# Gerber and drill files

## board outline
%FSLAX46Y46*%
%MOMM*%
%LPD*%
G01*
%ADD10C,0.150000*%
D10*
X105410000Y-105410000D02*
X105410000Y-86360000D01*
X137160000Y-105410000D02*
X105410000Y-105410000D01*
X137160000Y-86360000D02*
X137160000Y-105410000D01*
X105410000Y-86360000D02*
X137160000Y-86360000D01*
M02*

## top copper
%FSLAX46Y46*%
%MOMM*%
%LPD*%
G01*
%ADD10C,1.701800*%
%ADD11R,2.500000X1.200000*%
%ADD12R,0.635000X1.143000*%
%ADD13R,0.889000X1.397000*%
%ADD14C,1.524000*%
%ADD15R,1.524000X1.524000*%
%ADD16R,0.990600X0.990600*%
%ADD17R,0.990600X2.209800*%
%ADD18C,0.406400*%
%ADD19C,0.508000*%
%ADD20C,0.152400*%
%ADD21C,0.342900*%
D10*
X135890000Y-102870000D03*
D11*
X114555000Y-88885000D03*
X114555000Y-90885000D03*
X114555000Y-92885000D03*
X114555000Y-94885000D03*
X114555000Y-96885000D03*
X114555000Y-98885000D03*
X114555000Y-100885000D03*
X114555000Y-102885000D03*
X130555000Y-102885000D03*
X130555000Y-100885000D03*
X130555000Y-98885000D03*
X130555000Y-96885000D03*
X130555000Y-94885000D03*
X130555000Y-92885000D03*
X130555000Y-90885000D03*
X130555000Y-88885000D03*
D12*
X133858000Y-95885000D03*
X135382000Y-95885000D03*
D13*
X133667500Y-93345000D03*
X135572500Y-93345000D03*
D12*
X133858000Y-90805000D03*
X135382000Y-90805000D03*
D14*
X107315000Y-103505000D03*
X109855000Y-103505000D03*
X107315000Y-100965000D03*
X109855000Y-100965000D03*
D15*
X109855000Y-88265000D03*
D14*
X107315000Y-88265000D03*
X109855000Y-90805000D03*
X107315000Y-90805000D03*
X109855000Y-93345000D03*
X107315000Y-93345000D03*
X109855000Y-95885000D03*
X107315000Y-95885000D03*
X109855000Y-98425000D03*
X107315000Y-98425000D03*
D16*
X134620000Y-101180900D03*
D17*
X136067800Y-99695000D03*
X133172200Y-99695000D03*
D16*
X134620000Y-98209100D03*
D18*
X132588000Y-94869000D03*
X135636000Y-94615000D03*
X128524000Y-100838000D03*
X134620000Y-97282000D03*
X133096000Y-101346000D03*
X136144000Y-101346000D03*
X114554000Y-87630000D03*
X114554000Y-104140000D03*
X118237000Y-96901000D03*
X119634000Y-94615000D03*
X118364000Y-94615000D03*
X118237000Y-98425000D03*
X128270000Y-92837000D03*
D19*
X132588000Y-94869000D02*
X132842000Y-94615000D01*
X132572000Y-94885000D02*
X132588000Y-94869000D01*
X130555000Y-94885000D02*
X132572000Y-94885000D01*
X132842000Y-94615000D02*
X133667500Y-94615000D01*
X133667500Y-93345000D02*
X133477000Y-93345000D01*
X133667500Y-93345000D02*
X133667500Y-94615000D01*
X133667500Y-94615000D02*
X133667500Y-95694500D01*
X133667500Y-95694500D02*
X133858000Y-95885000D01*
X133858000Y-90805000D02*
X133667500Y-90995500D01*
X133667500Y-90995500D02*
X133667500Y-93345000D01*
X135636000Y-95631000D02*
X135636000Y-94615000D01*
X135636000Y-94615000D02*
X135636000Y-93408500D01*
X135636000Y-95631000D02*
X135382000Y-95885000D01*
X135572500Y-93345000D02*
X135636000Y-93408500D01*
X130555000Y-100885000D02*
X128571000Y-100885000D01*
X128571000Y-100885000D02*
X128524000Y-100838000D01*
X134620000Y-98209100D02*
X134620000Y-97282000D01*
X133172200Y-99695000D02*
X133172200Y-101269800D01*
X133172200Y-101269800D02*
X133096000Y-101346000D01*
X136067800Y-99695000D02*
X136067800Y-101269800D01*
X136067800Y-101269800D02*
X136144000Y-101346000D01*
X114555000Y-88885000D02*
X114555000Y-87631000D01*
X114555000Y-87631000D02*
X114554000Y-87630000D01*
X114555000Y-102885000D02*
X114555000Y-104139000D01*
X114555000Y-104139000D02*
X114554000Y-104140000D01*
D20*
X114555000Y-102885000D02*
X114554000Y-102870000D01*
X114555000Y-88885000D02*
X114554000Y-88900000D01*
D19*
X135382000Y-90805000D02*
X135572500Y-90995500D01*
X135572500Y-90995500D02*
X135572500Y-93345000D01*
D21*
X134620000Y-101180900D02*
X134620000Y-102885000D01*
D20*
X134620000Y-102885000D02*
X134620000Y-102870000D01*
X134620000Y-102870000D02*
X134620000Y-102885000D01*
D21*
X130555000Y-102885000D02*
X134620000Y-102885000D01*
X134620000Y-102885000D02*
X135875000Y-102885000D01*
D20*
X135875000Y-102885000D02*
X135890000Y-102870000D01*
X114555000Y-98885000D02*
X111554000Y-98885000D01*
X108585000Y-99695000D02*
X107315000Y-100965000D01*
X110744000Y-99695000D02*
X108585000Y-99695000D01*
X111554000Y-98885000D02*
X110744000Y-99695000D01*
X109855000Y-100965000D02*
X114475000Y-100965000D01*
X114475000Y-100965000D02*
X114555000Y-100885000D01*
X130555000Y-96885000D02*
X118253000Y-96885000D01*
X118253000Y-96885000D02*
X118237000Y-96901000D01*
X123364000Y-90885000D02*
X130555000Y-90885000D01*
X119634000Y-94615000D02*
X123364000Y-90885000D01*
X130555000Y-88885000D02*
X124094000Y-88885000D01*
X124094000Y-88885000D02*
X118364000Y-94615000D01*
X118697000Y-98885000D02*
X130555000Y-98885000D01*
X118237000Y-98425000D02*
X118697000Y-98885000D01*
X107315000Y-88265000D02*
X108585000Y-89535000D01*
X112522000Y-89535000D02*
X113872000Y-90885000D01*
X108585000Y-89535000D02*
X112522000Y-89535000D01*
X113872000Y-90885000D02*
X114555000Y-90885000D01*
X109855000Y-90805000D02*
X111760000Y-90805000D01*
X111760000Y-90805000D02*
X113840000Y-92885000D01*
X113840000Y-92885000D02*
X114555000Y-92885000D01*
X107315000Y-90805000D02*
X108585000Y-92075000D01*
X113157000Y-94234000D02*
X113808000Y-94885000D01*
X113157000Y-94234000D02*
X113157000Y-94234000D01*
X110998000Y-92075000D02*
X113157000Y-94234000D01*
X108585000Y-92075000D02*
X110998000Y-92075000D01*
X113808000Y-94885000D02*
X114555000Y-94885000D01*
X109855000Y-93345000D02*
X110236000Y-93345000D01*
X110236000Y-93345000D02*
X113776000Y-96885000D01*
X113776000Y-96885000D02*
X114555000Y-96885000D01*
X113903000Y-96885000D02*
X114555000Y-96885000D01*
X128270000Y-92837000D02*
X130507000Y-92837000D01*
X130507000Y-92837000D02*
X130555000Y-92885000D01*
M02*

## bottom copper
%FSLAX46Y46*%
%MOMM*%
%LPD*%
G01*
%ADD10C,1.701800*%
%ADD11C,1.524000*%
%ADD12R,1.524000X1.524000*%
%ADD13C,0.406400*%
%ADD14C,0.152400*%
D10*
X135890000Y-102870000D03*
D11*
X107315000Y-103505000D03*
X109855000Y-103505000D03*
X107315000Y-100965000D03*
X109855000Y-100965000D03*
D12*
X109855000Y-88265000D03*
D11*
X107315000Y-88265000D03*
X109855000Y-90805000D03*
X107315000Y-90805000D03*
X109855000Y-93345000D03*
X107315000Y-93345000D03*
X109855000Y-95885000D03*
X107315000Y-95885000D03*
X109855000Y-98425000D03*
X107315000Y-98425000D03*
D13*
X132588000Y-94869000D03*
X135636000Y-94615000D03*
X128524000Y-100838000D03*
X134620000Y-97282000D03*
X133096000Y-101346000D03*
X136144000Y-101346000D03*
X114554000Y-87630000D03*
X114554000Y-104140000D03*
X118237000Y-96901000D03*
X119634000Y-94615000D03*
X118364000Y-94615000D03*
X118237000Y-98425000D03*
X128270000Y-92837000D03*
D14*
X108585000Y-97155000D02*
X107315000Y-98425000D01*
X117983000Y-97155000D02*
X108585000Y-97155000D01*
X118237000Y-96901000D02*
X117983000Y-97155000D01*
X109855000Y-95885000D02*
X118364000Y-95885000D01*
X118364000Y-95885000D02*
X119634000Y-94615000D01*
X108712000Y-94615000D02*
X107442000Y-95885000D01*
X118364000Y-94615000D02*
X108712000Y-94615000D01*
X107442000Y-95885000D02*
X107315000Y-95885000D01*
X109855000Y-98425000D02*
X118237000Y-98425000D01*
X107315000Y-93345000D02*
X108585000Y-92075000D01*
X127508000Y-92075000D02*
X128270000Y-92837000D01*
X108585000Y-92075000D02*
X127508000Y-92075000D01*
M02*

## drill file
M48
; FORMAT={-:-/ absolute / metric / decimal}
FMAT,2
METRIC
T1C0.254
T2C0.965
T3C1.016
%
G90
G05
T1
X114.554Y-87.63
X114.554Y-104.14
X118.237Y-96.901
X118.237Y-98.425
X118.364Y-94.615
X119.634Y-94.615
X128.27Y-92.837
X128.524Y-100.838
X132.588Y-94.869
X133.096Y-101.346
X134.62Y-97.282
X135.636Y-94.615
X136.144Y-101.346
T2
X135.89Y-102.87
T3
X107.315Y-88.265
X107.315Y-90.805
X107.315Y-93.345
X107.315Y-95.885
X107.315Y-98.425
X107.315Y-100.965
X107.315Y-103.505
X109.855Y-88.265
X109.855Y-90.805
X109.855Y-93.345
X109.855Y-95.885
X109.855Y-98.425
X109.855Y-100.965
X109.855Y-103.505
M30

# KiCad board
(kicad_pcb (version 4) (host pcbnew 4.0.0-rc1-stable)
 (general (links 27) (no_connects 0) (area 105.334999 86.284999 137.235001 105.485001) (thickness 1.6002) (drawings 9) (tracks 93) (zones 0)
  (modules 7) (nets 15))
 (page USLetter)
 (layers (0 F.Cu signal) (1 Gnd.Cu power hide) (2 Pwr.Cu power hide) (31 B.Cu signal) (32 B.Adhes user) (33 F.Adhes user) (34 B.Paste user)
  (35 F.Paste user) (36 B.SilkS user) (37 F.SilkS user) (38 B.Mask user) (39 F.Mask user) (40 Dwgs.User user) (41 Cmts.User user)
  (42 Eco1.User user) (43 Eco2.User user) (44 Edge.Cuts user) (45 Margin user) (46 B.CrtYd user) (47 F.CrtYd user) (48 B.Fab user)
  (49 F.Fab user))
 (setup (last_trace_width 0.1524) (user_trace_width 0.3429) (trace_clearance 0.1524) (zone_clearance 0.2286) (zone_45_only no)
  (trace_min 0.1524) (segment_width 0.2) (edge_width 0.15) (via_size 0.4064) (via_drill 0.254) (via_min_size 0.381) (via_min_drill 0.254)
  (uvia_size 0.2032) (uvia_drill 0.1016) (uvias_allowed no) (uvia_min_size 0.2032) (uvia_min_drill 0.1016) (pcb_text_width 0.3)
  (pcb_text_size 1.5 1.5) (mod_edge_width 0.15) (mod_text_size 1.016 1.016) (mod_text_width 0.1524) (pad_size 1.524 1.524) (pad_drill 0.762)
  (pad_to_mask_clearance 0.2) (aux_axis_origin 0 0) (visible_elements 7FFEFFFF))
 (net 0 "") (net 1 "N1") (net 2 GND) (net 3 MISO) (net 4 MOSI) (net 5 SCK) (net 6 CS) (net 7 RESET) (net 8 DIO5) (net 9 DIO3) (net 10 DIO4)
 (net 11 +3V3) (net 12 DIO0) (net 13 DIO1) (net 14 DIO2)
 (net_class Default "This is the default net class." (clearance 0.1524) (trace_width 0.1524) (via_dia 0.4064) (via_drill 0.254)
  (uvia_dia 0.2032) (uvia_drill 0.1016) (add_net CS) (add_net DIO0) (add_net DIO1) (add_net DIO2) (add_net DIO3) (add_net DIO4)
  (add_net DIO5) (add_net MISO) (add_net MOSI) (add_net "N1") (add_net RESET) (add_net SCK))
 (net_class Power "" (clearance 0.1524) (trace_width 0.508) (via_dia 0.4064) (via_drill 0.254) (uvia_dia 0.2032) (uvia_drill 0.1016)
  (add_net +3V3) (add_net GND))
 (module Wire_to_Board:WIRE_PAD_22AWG (layer F.Cu) (at 135.89 102.87)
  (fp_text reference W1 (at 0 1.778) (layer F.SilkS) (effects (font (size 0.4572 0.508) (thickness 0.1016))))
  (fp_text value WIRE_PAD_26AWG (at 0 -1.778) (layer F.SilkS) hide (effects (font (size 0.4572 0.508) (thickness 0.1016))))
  (pad 1 thru_hole circle (at 0 0) (size 1.7018 1.7018) (drill 0.9652) (layers *.Cu *.Mask F.SilkS) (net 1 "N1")))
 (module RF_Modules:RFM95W (layer F.Cu) (at 122.555 95.885)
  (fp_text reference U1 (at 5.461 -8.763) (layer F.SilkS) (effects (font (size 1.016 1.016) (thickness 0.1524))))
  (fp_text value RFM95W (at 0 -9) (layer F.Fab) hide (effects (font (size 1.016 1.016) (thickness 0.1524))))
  (pad 1 smd rect (at -8 -7) (size 2.5 1.2) (layers F.Cu F.Paste F.Mask) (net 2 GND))
  (pad 2 smd rect (at -8 -5) (size 2.5 1.2) (layers F.Cu F.Paste F.Mask) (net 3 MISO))
  (pad 3 smd rect (at -8 -3) (size 2.5 1.2) (layers F.Cu F.Paste F.Mask) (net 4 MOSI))
  (pad 4 smd rect (at -8 -1) (size 2.5 1.2) (layers F.Cu F.Paste F.Mask) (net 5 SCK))
  (pad 5 smd rect (at -8 1) (size 2.5 1.2) (layers F.Cu F.Paste F.Mask) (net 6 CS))
  (pad 6 smd rect (at -8 3) (size 2.5 1.2) (layers F.Cu F.Paste F.Mask) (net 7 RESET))
  (pad 7 smd rect (at -8 5) (size 2.5 1.2) (layers F.Cu F.Paste F.Mask) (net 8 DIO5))
  (pad 8 smd rect (at -8 7) (size 2.5 1.2) (layers F.Cu F.Paste F.Mask) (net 2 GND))
  (pad 9 smd rect (at 8 7) (size 2.5 1.2) (layers F.Cu F.Paste F.Mask) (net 1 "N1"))
  (pad 10 smd rect (at 8 5) (size 2.5 1.2) (layers F.Cu F.Paste F.Mask) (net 2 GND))
  (pad 11 smd rect (at 8 3) (size 2.5 1.2) (layers F.Cu F.Paste F.Mask) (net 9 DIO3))
  (pad 12 smd rect (at 8 1) (size 2.5 1.2) (layers F.Cu F.Paste F.Mask) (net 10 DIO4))
  (pad 13 smd rect (at 8 -1) (size 2.5 1.2) (layers F.Cu F.Paste F.Mask) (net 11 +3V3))
  (pad 14 smd rect (at 8 -3) (size 2.5 1.2) (layers F.Cu F.Paste F.Mask) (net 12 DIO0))
  (pad 15 smd rect (at 8 -5) (size 2.5 1.2) (layers F.Cu F.Paste F.Mask) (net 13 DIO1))
  (pad 16 smd rect (at 8 -7) (size 2.5 1.2) (layers F.Cu F.Paste F.Mask) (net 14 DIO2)))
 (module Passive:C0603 (layer F.Cu) (at 134.62 95.885)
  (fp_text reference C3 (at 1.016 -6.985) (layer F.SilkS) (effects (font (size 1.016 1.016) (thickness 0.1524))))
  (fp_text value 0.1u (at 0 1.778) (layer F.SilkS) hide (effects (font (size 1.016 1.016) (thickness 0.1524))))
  (pad 1 smd rect (at -0.762 0) (size 0.635 1.143) (layers F.Cu F.Paste F.Mask) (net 11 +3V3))
  (pad 2 smd rect (at 0.762 0) (size 0.635 1.143) (layers F.Cu F.Paste F.Mask) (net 2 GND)))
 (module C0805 (layer F.Cu) (at 134.62 93.345)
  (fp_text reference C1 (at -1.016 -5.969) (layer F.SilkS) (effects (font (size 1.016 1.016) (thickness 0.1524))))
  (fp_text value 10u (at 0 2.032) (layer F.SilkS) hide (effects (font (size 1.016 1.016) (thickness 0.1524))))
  (pad 1 smd rect (at -0.9525 0) (size 0.889 1.397) (layers F.Cu F.Paste F.Mask) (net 11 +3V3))
  (pad 2 smd rect (at 0.9525 0) (size 0.889 1.397) (layers F.Cu F.Paste F.Mask) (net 2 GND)))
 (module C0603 (layer F.Cu) (at 134.62 90.805)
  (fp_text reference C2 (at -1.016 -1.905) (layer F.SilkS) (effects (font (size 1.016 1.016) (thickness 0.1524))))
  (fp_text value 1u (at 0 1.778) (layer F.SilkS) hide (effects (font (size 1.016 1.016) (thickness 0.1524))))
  (pad 1 smd rect (at -0.762 0) (size 0.635 1.143) (layers F.Cu F.Paste F.Mask) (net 11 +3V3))
  (pad 2 smd rect (at 0.762 0) (size 0.635 1.143) (layers F.Cu F.Paste F.Mask) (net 2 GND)))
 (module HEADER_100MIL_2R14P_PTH (layer B.Cu) (at 108.585 95.885 270)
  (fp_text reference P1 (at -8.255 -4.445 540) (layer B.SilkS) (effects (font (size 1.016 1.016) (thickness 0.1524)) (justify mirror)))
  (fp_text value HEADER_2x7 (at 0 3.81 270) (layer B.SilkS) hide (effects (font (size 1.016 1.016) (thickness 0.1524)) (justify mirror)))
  (pad 14 thru_hole circle (at 7.62 1.27 270) (size 1.524 1.524) (drill 1.016) (layers *.Cu *.Mask B.SilkS) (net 2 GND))
  (pad 13 thru_hole circle (at 7.62 -1.27 270) (size 1.524 1.524) (drill 1.016) (layers *.Cu *.Mask B.SilkS) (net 11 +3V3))
  (pad 12 thru_hole circle (at 5.08 1.27 270) (size 1.524 1.524) (drill 1.016) (layers *.Cu *.Mask B.SilkS) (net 7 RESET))
  (pad 11 thru_hole circle (at 5.08 -1.27 270) (size 1.524 1.524) (drill 1.016) (layers *.Cu *.Mask B.SilkS) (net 8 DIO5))
  (pad 1 thru_hole rect (at -7.62 -1.27 270) (size 1.524 1.524) (drill 1.016) (layers *.Cu *.Mask B.SilkS) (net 2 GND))
  (pad 2 thru_hole circle (at -7.62 1.27 270) (size 1.524 1.524) (drill 1.016) (layers *.Cu *.Mask B.SilkS) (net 3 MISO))
  (pad 3 thru_hole circle (at -5.08 -1.27 270) (size 1.524 1.524) (drill 1.016) (layers *.Cu *.Mask B.SilkS) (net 4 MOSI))
  (pad 4 thru_hole circle (at -5.08 1.27 270) (size 1.524 1.524) (drill 1.016) (layers *.Cu *.Mask B.SilkS) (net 5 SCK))
  (pad 5 thru_hole circle (at -2.54 -1.27 270) (size 1.524 1.524) (drill 1.016) (layers *.Cu *.Mask B.SilkS) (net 6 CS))
  (pad 6 thru_hole circle (at -2.54 1.27 270) (size 1.524 1.524) (drill 1.016) (layers *.Cu *.Mask B.SilkS) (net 12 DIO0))
  (pad 7 thru_hole circle (at 0 -1.27 270) (size 1.524 1.524) (drill 1.016) (layers *.Cu *.Mask B.SilkS) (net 13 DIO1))
  (pad 8 thru_hole circle (at 0 1.27 270) (size 1.524 1.524) (drill 1.016) (layers *.Cu *.Mask B.SilkS) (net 14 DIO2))
  (pad 9 thru_hole circle (at 2.54 -1.27 270) (size 1.524 1.524) (drill 1.016) (layers *.Cu *.Mask B.SilkS) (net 9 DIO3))
  (pad 10 thru_hole circle (at 2.54 1.27 270) (size 1.524 1.524) (drill 1.016) (layers *.Cu *.Mask B.SilkS) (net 10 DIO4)))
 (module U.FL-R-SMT (layer F.Cu) (at 134.62 99.695)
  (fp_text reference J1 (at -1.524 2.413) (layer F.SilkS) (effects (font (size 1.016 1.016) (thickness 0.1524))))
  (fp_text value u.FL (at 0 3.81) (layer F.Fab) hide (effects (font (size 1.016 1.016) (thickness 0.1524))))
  (pad 1 smd rect (at 0 1.4859) (size 0.9906 0.9906) (layers F.Cu F.Paste F.Mask) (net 1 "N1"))
  (pad 4 smd rect (at 1.4478 0) (size 0.9906 2.2098) (layers F.Cu F.Paste F.Mask) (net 2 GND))
  (pad 2 smd rect (at -1.4478 0) (size 0.9906 2.2098) (layers F.Cu F.Paste F.Mask) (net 2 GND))
  (pad 3 smd rect (at 0 -1.4859) (size 0.9906 0.9906) (layers F.Cu F.Paste F.Mask) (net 2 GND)))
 (gr_line (start 105.41 105.41) (end 105.41 86.36) (angle 90) (layer Edge.Cuts) (width 0.15))
 (gr_line (start 137.16 105.41) (end 105.41 105.41) (angle 90) (layer Edge.Cuts) (width 0.15))
 (gr_line (start 137.16 86.36) (end 137.16 105.41) (angle 90) (layer Edge.Cuts) (width 0.15))
 (gr_line (start 105.41 86.36) (end 137.16 86.36) (angle 90) (layer Edge.Cuts) (width 0.15))
 (segment (start 132.588 94.869) (end 132.842 94.615) (width 0.508) (layer F.Cu) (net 11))
 (segment (start 132.572 94.885) (end 132.588 94.869) (width 0.508) (layer F.Cu) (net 11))
 (via (at 132.588 94.869) (size 0.4064) (drill 0.254) (layers F.Cu B.Cu) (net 11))
 (segment (start 130.555 94.885) (end 132.572 94.885) (width 0.508) (layer F.Cu) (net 11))
 (segment (start 132.842 94.615) (end 133.6675 94.615) (width 0.508) (layer F.Cu) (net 11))
 (segment (start 133.6675 93.345) (end 133.477 93.345) (width 0.508) (layer F.Cu) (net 11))
 (segment (start 133.6675 93.345) (end 133.6675 94.615) (width 0.508) (layer F.Cu) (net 11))
 (segment (start 133.6675 94.615) (end 133.6675 95.6945) (width 0.508) (layer F.Cu) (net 11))
 (segment (start 133.6675 95.6945) (end 133.858 95.885) (width 0.508) (layer F.Cu) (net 11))
 (segment (start 133.858 90.805) (end 133.6675 90.9955) (width 0.508) (layer F.Cu) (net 11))
 (segment (start 133.6675 90.9955) (end 133.6675 93.345) (width 0.508) (layer F.Cu) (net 11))
 (segment (start 135.636 95.631) (end 135.636 94.615) (width 0.508) (layer F.Cu) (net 2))
 (via (at 135.636 94.615) (size 0.4064) (drill 0.254) (layers F.Cu B.Cu) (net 2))
 (segment (start 135.636 94.615) (end 135.636 93.4085) (width 0.508) (layer F.Cu) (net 2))
 (segment (start 135.636 95.631) (end 135.382 95.885) (width 0.508) (layer F.Cu) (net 2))
 (segment (start 135.5725 93.345) (end 135.636 93.4085) (width 0.508) (layer F.Cu) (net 2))
 (segment (start 130.555 100.885) (end 128.571 100.885) (width 0.508) (layer F.Cu) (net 2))
 (via (at 128.524 100.838) (size 0.4064) (drill 0.254) (layers F.Cu B.Cu) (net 2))
 (segment (start 128.571 100.885) (end 128.524 100.838) (width 0.508) (layer F.Cu) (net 2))
 (segment (start 134.62 98.2091) (end 134.62 97.282) (width 0.508) (layer F.Cu) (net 2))
 (via (at 134.62 97.282) (size 0.4064) (drill 0.254) (layers F.Cu B.Cu) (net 2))
 (segment (start 133.1722 99.695) (end 133.1722 101.2698) (width 0.508) (layer F.Cu) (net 2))
 (via (at 133.096 101.346) (size 0.4064) (drill 0.254) (layers F.Cu B.Cu) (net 2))
 (segment (start 133.1722 101.2698) (end 133.096 101.346) (width 0.508) (layer F.Cu) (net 2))
 (segment (start 136.0678 99.695) (end 136.0678 101.2698) (width 0.508) (layer F.Cu) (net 2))
 (via (at 136.144 101.346) (size 0.4064) (drill 0.254) (layers F.Cu B.Cu) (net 2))
 (segment (start 136.0678 101.2698) (end 136.144 101.346) (width 0.508) (layer F.Cu) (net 2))
 (segment (start 114.555 88.885) (end 114.555 87.631) (width 0.508) (layer F.Cu) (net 2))
 (via (at 114.554 87.63) (size 0.4064) (drill 0.254) (layers F.Cu B.Cu) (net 2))
 (segment (start 114.555 87.631) (end 114.554 87.63) (width 0.508) (layer F.Cu) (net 2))
 (segment (start 114.555 102.885) (end 114.555 104.139) (width 0.508) (layer F.Cu) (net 2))
 (via (at 114.554 104.14) (size 0.4064) (drill 0.254) (layers F.Cu B.Cu) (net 2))
 (segment (start 114.555 104.139) (end 114.554 104.14) (width 0.508) (layer F.Cu) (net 2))
 (segment (start 114.555 102.885) (end 114.554 102.87) (width 0.1524) (layer F.Cu) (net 2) (status 80000))
 (segment (start 114.555 88.885) (end 114.554 88.9) (width 0.1524) (layer F.Cu) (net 2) (status 80000))
 (segment (start 135.382 90.805) (end 135.5725 90.9955) (width 0.508) (layer F.Cu) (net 2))
 (segment (start 135.5725 90.9955) (end 135.5725 93.345) (width 0.508) (layer F.Cu) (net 2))
 (segment (start 134.62 101.1809) (end 134.62 102.885) (width 0.3429) (layer F.Cu) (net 1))
 (segment (start 134.62 102.885) (end 134.62 102.87) (width 0.1524) (layer F.Cu) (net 1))
 (segment (start 134.62 102.87) (end 134.62 102.885) (width 0.1524) (layer F.Cu) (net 1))
 (segment (start 130.555 102.885) (end 134.62 102.885) (width 0.3429) (layer F.Cu) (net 1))
 (segment (start 134.62 102.885) (end 135.875 102.885) (width 0.3429) (layer F.Cu) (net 1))
 (segment (start 135.875 102.885) (end 135.89 102.87) (width 0.1524) (layer F.Cu) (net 1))
 (segment (start 114.555 98.885) (end 111.554 98.885) (width 0.1524) (layer F.Cu) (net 7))
 (segment (start 108.585 99.695) (end 107.315 100.965) (width 0.1524) (layer F.Cu) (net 7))
 (segment (start 110.744 99.695) (end 108.585 99.695) (width 0.1524) (layer F.Cu) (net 7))
 (segment (start 111.554 98.885) (end 110.744 99.695) (width 0.1524) (layer F.Cu) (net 7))
 (segment (start 109.855 100.965) (end 114.475 100.965) (width 0.1524) (layer F.Cu) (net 8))
 (segment (start 114.475 100.965) (end 114.555 100.885) (width 0.1524) (layer F.Cu) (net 8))
 (segment (start 130.555 96.885) (end 118.253 96.885) (width 0.1524) (layer F.Cu) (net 10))
 (segment (start 108.585 97.155) (end 107.315 98.425) (width 0.1524) (layer B.Cu) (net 10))
 (segment (start 117.983 97.155) (end 108.585 97.155) (width 0.1524) (layer B.Cu) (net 10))
 (segment (start 118.237 96.901) (end 117.983 97.155) (width 0.1524) (layer B.Cu) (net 10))
 (via (at 118.237 96.901) (size 0.4064) (drill 0.254) (layers F.Cu B.Cu) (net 10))
 (segment (start 118.253 96.885) (end 118.237 96.901) (width 0.1524) (layer F.Cu) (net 10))
 (segment (start 109.855 95.885) (end 118.364 95.885) (width 0.1524) (layer B.Cu) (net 13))
 (segment (start 123.364 90.885) (end 130.555 90.885) (width 0.1524) (layer F.Cu) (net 13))
 (segment (start 119.634 94.615) (end 123.364 90.885) (width 0.1524) (layer F.Cu) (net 13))
 (via (at 119.634 94.615) (size 0.4064) (drill 0.254) (layers F.Cu B.Cu) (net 13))
 (segment (start 118.364 95.885) (end 119.634 94.615) (width 0.1524) (layer B.Cu) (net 13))
 (segment (start 130.555 88.885) (end 124.094 88.885) (width 0.1524) (layer F.Cu) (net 14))
 (segment (start 108.712 94.615) (end 107.442 95.885) (width 0.1524) (layer B.Cu) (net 14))
 (segment (start 118.364 94.615) (end 108.712 94.615) (width 0.1524) (layer B.Cu) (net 14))
 (via (at 118.364 94.615) (size 0.4064) (drill 0.254) (layers F.Cu B.Cu) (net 14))
 (segment (start 124.094 88.885) (end 118.364 94.615) (width 0.1524) (layer F.Cu) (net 14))
 (segment (start 107.442 95.885) (end 107.315 95.885) (width 0.1524) (layer B.Cu) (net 14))
 (segment (start 109.855 98.425) (end 118.237 98.425) (width 0.1524) (layer B.Cu) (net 9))
 (segment (start 118.697 98.885) (end 130.555 98.885) (width 0.1524) (layer F.Cu) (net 9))
 (segment (start 118.237 98.425) (end 118.697 98.885) (width 0.1524) (layer F.Cu) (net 9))
 (via (at 118.237 98.425) (size 0.4064) (drill 0.254) (layers F.Cu B.Cu) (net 9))
 (segment (start 107.315 88.265) (end 108.585 89.535) (width 0.1524) (layer F.Cu) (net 3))
 (segment (start 112.522 89.535) (end 113.872 90.885) (width 0.1524) (layer F.Cu) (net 3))
 (segment (start 108.585 89.535) (end 112.522 89.535) (width 0.1524) (layer F.Cu) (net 3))
 (segment (start 113.872 90.885) (end 114.555 90.885) (width 0.1524) (layer F.Cu) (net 3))
 (segment (start 109.855 90.805) (end 111.76 90.805) (width 0.1524) (layer F.Cu) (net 4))
 (segment (start 111.76 90.805) (end 113.84 92.885) (width 0.1524) (layer F.Cu) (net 4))
 (segment (start 113.84 92.885) (end 114.555 92.885) (width 0.1524) (layer F.Cu) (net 4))
 (segment (start 107.315 90.805) (end 108.585 92.075) (width 0.1524) (layer F.Cu) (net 5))
 (segment (start 113.157 94.234) (end 113.808 94.885) (width 0.1524) (layer F.Cu) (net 5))
 (segment (start 113.157 94.234) (end 113.157 94.234) (width 0.1524) (layer F.Cu) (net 5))
 (segment (start 110.998 92.075) (end 113.157 94.234) (width 0.1524) (layer F.Cu) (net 5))
 (segment (start 108.585 92.075) (end 110.998 92.075) (width 0.1524) (layer F.Cu) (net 5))
 (segment (start 113.808 94.885) (end 114.555 94.885) (width 0.1524) (layer F.Cu) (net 5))
 (segment (start 109.855 93.345) (end 110.236 93.345) (width 0.1524) (layer F.Cu) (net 6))
 (segment (start 110.236 93.345) (end 113.776 96.885) (width 0.1524) (layer F.Cu) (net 6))
 (segment (start 113.776 96.885) (end 114.555 96.885) (width 0.1524) (layer F.Cu) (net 6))
 (segment (start 113.903 96.885) (end 114.555 96.885) (width 0.1524) (layer F.Cu) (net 6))
 (segment (start 107.315 93.345) (end 108.585 92.075) (width 0.1524) (layer B.Cu) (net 12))
 (segment (start 128.27 92.837) (end 130.507 92.837) (width 0.1524) (layer F.Cu) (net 12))
 (via (at 128.27 92.837) (size 0.4064) (drill 0.254) (layers F.Cu B.Cu) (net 12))
 (segment (start 127.508 92.075) (end 128.27 92.837) (width 0.1524) (layer B.Cu) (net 12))
 (segment (start 108.585 92.075) (end 127.508 92.075) (width 0.1524) (layer B.Cu) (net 12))
 (segment (start 130.507 92.837) (end 130.555 92.885) (width 0.1524) (layer F.Cu) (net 12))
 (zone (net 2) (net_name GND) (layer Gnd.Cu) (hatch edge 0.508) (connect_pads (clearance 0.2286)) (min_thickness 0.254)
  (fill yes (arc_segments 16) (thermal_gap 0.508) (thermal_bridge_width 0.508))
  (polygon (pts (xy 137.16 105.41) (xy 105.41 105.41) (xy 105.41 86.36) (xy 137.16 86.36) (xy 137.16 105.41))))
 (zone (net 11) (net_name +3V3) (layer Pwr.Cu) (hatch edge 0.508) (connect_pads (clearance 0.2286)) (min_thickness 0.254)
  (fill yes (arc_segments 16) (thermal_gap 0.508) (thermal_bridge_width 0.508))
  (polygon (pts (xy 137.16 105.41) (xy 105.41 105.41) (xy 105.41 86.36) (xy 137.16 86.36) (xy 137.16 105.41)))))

